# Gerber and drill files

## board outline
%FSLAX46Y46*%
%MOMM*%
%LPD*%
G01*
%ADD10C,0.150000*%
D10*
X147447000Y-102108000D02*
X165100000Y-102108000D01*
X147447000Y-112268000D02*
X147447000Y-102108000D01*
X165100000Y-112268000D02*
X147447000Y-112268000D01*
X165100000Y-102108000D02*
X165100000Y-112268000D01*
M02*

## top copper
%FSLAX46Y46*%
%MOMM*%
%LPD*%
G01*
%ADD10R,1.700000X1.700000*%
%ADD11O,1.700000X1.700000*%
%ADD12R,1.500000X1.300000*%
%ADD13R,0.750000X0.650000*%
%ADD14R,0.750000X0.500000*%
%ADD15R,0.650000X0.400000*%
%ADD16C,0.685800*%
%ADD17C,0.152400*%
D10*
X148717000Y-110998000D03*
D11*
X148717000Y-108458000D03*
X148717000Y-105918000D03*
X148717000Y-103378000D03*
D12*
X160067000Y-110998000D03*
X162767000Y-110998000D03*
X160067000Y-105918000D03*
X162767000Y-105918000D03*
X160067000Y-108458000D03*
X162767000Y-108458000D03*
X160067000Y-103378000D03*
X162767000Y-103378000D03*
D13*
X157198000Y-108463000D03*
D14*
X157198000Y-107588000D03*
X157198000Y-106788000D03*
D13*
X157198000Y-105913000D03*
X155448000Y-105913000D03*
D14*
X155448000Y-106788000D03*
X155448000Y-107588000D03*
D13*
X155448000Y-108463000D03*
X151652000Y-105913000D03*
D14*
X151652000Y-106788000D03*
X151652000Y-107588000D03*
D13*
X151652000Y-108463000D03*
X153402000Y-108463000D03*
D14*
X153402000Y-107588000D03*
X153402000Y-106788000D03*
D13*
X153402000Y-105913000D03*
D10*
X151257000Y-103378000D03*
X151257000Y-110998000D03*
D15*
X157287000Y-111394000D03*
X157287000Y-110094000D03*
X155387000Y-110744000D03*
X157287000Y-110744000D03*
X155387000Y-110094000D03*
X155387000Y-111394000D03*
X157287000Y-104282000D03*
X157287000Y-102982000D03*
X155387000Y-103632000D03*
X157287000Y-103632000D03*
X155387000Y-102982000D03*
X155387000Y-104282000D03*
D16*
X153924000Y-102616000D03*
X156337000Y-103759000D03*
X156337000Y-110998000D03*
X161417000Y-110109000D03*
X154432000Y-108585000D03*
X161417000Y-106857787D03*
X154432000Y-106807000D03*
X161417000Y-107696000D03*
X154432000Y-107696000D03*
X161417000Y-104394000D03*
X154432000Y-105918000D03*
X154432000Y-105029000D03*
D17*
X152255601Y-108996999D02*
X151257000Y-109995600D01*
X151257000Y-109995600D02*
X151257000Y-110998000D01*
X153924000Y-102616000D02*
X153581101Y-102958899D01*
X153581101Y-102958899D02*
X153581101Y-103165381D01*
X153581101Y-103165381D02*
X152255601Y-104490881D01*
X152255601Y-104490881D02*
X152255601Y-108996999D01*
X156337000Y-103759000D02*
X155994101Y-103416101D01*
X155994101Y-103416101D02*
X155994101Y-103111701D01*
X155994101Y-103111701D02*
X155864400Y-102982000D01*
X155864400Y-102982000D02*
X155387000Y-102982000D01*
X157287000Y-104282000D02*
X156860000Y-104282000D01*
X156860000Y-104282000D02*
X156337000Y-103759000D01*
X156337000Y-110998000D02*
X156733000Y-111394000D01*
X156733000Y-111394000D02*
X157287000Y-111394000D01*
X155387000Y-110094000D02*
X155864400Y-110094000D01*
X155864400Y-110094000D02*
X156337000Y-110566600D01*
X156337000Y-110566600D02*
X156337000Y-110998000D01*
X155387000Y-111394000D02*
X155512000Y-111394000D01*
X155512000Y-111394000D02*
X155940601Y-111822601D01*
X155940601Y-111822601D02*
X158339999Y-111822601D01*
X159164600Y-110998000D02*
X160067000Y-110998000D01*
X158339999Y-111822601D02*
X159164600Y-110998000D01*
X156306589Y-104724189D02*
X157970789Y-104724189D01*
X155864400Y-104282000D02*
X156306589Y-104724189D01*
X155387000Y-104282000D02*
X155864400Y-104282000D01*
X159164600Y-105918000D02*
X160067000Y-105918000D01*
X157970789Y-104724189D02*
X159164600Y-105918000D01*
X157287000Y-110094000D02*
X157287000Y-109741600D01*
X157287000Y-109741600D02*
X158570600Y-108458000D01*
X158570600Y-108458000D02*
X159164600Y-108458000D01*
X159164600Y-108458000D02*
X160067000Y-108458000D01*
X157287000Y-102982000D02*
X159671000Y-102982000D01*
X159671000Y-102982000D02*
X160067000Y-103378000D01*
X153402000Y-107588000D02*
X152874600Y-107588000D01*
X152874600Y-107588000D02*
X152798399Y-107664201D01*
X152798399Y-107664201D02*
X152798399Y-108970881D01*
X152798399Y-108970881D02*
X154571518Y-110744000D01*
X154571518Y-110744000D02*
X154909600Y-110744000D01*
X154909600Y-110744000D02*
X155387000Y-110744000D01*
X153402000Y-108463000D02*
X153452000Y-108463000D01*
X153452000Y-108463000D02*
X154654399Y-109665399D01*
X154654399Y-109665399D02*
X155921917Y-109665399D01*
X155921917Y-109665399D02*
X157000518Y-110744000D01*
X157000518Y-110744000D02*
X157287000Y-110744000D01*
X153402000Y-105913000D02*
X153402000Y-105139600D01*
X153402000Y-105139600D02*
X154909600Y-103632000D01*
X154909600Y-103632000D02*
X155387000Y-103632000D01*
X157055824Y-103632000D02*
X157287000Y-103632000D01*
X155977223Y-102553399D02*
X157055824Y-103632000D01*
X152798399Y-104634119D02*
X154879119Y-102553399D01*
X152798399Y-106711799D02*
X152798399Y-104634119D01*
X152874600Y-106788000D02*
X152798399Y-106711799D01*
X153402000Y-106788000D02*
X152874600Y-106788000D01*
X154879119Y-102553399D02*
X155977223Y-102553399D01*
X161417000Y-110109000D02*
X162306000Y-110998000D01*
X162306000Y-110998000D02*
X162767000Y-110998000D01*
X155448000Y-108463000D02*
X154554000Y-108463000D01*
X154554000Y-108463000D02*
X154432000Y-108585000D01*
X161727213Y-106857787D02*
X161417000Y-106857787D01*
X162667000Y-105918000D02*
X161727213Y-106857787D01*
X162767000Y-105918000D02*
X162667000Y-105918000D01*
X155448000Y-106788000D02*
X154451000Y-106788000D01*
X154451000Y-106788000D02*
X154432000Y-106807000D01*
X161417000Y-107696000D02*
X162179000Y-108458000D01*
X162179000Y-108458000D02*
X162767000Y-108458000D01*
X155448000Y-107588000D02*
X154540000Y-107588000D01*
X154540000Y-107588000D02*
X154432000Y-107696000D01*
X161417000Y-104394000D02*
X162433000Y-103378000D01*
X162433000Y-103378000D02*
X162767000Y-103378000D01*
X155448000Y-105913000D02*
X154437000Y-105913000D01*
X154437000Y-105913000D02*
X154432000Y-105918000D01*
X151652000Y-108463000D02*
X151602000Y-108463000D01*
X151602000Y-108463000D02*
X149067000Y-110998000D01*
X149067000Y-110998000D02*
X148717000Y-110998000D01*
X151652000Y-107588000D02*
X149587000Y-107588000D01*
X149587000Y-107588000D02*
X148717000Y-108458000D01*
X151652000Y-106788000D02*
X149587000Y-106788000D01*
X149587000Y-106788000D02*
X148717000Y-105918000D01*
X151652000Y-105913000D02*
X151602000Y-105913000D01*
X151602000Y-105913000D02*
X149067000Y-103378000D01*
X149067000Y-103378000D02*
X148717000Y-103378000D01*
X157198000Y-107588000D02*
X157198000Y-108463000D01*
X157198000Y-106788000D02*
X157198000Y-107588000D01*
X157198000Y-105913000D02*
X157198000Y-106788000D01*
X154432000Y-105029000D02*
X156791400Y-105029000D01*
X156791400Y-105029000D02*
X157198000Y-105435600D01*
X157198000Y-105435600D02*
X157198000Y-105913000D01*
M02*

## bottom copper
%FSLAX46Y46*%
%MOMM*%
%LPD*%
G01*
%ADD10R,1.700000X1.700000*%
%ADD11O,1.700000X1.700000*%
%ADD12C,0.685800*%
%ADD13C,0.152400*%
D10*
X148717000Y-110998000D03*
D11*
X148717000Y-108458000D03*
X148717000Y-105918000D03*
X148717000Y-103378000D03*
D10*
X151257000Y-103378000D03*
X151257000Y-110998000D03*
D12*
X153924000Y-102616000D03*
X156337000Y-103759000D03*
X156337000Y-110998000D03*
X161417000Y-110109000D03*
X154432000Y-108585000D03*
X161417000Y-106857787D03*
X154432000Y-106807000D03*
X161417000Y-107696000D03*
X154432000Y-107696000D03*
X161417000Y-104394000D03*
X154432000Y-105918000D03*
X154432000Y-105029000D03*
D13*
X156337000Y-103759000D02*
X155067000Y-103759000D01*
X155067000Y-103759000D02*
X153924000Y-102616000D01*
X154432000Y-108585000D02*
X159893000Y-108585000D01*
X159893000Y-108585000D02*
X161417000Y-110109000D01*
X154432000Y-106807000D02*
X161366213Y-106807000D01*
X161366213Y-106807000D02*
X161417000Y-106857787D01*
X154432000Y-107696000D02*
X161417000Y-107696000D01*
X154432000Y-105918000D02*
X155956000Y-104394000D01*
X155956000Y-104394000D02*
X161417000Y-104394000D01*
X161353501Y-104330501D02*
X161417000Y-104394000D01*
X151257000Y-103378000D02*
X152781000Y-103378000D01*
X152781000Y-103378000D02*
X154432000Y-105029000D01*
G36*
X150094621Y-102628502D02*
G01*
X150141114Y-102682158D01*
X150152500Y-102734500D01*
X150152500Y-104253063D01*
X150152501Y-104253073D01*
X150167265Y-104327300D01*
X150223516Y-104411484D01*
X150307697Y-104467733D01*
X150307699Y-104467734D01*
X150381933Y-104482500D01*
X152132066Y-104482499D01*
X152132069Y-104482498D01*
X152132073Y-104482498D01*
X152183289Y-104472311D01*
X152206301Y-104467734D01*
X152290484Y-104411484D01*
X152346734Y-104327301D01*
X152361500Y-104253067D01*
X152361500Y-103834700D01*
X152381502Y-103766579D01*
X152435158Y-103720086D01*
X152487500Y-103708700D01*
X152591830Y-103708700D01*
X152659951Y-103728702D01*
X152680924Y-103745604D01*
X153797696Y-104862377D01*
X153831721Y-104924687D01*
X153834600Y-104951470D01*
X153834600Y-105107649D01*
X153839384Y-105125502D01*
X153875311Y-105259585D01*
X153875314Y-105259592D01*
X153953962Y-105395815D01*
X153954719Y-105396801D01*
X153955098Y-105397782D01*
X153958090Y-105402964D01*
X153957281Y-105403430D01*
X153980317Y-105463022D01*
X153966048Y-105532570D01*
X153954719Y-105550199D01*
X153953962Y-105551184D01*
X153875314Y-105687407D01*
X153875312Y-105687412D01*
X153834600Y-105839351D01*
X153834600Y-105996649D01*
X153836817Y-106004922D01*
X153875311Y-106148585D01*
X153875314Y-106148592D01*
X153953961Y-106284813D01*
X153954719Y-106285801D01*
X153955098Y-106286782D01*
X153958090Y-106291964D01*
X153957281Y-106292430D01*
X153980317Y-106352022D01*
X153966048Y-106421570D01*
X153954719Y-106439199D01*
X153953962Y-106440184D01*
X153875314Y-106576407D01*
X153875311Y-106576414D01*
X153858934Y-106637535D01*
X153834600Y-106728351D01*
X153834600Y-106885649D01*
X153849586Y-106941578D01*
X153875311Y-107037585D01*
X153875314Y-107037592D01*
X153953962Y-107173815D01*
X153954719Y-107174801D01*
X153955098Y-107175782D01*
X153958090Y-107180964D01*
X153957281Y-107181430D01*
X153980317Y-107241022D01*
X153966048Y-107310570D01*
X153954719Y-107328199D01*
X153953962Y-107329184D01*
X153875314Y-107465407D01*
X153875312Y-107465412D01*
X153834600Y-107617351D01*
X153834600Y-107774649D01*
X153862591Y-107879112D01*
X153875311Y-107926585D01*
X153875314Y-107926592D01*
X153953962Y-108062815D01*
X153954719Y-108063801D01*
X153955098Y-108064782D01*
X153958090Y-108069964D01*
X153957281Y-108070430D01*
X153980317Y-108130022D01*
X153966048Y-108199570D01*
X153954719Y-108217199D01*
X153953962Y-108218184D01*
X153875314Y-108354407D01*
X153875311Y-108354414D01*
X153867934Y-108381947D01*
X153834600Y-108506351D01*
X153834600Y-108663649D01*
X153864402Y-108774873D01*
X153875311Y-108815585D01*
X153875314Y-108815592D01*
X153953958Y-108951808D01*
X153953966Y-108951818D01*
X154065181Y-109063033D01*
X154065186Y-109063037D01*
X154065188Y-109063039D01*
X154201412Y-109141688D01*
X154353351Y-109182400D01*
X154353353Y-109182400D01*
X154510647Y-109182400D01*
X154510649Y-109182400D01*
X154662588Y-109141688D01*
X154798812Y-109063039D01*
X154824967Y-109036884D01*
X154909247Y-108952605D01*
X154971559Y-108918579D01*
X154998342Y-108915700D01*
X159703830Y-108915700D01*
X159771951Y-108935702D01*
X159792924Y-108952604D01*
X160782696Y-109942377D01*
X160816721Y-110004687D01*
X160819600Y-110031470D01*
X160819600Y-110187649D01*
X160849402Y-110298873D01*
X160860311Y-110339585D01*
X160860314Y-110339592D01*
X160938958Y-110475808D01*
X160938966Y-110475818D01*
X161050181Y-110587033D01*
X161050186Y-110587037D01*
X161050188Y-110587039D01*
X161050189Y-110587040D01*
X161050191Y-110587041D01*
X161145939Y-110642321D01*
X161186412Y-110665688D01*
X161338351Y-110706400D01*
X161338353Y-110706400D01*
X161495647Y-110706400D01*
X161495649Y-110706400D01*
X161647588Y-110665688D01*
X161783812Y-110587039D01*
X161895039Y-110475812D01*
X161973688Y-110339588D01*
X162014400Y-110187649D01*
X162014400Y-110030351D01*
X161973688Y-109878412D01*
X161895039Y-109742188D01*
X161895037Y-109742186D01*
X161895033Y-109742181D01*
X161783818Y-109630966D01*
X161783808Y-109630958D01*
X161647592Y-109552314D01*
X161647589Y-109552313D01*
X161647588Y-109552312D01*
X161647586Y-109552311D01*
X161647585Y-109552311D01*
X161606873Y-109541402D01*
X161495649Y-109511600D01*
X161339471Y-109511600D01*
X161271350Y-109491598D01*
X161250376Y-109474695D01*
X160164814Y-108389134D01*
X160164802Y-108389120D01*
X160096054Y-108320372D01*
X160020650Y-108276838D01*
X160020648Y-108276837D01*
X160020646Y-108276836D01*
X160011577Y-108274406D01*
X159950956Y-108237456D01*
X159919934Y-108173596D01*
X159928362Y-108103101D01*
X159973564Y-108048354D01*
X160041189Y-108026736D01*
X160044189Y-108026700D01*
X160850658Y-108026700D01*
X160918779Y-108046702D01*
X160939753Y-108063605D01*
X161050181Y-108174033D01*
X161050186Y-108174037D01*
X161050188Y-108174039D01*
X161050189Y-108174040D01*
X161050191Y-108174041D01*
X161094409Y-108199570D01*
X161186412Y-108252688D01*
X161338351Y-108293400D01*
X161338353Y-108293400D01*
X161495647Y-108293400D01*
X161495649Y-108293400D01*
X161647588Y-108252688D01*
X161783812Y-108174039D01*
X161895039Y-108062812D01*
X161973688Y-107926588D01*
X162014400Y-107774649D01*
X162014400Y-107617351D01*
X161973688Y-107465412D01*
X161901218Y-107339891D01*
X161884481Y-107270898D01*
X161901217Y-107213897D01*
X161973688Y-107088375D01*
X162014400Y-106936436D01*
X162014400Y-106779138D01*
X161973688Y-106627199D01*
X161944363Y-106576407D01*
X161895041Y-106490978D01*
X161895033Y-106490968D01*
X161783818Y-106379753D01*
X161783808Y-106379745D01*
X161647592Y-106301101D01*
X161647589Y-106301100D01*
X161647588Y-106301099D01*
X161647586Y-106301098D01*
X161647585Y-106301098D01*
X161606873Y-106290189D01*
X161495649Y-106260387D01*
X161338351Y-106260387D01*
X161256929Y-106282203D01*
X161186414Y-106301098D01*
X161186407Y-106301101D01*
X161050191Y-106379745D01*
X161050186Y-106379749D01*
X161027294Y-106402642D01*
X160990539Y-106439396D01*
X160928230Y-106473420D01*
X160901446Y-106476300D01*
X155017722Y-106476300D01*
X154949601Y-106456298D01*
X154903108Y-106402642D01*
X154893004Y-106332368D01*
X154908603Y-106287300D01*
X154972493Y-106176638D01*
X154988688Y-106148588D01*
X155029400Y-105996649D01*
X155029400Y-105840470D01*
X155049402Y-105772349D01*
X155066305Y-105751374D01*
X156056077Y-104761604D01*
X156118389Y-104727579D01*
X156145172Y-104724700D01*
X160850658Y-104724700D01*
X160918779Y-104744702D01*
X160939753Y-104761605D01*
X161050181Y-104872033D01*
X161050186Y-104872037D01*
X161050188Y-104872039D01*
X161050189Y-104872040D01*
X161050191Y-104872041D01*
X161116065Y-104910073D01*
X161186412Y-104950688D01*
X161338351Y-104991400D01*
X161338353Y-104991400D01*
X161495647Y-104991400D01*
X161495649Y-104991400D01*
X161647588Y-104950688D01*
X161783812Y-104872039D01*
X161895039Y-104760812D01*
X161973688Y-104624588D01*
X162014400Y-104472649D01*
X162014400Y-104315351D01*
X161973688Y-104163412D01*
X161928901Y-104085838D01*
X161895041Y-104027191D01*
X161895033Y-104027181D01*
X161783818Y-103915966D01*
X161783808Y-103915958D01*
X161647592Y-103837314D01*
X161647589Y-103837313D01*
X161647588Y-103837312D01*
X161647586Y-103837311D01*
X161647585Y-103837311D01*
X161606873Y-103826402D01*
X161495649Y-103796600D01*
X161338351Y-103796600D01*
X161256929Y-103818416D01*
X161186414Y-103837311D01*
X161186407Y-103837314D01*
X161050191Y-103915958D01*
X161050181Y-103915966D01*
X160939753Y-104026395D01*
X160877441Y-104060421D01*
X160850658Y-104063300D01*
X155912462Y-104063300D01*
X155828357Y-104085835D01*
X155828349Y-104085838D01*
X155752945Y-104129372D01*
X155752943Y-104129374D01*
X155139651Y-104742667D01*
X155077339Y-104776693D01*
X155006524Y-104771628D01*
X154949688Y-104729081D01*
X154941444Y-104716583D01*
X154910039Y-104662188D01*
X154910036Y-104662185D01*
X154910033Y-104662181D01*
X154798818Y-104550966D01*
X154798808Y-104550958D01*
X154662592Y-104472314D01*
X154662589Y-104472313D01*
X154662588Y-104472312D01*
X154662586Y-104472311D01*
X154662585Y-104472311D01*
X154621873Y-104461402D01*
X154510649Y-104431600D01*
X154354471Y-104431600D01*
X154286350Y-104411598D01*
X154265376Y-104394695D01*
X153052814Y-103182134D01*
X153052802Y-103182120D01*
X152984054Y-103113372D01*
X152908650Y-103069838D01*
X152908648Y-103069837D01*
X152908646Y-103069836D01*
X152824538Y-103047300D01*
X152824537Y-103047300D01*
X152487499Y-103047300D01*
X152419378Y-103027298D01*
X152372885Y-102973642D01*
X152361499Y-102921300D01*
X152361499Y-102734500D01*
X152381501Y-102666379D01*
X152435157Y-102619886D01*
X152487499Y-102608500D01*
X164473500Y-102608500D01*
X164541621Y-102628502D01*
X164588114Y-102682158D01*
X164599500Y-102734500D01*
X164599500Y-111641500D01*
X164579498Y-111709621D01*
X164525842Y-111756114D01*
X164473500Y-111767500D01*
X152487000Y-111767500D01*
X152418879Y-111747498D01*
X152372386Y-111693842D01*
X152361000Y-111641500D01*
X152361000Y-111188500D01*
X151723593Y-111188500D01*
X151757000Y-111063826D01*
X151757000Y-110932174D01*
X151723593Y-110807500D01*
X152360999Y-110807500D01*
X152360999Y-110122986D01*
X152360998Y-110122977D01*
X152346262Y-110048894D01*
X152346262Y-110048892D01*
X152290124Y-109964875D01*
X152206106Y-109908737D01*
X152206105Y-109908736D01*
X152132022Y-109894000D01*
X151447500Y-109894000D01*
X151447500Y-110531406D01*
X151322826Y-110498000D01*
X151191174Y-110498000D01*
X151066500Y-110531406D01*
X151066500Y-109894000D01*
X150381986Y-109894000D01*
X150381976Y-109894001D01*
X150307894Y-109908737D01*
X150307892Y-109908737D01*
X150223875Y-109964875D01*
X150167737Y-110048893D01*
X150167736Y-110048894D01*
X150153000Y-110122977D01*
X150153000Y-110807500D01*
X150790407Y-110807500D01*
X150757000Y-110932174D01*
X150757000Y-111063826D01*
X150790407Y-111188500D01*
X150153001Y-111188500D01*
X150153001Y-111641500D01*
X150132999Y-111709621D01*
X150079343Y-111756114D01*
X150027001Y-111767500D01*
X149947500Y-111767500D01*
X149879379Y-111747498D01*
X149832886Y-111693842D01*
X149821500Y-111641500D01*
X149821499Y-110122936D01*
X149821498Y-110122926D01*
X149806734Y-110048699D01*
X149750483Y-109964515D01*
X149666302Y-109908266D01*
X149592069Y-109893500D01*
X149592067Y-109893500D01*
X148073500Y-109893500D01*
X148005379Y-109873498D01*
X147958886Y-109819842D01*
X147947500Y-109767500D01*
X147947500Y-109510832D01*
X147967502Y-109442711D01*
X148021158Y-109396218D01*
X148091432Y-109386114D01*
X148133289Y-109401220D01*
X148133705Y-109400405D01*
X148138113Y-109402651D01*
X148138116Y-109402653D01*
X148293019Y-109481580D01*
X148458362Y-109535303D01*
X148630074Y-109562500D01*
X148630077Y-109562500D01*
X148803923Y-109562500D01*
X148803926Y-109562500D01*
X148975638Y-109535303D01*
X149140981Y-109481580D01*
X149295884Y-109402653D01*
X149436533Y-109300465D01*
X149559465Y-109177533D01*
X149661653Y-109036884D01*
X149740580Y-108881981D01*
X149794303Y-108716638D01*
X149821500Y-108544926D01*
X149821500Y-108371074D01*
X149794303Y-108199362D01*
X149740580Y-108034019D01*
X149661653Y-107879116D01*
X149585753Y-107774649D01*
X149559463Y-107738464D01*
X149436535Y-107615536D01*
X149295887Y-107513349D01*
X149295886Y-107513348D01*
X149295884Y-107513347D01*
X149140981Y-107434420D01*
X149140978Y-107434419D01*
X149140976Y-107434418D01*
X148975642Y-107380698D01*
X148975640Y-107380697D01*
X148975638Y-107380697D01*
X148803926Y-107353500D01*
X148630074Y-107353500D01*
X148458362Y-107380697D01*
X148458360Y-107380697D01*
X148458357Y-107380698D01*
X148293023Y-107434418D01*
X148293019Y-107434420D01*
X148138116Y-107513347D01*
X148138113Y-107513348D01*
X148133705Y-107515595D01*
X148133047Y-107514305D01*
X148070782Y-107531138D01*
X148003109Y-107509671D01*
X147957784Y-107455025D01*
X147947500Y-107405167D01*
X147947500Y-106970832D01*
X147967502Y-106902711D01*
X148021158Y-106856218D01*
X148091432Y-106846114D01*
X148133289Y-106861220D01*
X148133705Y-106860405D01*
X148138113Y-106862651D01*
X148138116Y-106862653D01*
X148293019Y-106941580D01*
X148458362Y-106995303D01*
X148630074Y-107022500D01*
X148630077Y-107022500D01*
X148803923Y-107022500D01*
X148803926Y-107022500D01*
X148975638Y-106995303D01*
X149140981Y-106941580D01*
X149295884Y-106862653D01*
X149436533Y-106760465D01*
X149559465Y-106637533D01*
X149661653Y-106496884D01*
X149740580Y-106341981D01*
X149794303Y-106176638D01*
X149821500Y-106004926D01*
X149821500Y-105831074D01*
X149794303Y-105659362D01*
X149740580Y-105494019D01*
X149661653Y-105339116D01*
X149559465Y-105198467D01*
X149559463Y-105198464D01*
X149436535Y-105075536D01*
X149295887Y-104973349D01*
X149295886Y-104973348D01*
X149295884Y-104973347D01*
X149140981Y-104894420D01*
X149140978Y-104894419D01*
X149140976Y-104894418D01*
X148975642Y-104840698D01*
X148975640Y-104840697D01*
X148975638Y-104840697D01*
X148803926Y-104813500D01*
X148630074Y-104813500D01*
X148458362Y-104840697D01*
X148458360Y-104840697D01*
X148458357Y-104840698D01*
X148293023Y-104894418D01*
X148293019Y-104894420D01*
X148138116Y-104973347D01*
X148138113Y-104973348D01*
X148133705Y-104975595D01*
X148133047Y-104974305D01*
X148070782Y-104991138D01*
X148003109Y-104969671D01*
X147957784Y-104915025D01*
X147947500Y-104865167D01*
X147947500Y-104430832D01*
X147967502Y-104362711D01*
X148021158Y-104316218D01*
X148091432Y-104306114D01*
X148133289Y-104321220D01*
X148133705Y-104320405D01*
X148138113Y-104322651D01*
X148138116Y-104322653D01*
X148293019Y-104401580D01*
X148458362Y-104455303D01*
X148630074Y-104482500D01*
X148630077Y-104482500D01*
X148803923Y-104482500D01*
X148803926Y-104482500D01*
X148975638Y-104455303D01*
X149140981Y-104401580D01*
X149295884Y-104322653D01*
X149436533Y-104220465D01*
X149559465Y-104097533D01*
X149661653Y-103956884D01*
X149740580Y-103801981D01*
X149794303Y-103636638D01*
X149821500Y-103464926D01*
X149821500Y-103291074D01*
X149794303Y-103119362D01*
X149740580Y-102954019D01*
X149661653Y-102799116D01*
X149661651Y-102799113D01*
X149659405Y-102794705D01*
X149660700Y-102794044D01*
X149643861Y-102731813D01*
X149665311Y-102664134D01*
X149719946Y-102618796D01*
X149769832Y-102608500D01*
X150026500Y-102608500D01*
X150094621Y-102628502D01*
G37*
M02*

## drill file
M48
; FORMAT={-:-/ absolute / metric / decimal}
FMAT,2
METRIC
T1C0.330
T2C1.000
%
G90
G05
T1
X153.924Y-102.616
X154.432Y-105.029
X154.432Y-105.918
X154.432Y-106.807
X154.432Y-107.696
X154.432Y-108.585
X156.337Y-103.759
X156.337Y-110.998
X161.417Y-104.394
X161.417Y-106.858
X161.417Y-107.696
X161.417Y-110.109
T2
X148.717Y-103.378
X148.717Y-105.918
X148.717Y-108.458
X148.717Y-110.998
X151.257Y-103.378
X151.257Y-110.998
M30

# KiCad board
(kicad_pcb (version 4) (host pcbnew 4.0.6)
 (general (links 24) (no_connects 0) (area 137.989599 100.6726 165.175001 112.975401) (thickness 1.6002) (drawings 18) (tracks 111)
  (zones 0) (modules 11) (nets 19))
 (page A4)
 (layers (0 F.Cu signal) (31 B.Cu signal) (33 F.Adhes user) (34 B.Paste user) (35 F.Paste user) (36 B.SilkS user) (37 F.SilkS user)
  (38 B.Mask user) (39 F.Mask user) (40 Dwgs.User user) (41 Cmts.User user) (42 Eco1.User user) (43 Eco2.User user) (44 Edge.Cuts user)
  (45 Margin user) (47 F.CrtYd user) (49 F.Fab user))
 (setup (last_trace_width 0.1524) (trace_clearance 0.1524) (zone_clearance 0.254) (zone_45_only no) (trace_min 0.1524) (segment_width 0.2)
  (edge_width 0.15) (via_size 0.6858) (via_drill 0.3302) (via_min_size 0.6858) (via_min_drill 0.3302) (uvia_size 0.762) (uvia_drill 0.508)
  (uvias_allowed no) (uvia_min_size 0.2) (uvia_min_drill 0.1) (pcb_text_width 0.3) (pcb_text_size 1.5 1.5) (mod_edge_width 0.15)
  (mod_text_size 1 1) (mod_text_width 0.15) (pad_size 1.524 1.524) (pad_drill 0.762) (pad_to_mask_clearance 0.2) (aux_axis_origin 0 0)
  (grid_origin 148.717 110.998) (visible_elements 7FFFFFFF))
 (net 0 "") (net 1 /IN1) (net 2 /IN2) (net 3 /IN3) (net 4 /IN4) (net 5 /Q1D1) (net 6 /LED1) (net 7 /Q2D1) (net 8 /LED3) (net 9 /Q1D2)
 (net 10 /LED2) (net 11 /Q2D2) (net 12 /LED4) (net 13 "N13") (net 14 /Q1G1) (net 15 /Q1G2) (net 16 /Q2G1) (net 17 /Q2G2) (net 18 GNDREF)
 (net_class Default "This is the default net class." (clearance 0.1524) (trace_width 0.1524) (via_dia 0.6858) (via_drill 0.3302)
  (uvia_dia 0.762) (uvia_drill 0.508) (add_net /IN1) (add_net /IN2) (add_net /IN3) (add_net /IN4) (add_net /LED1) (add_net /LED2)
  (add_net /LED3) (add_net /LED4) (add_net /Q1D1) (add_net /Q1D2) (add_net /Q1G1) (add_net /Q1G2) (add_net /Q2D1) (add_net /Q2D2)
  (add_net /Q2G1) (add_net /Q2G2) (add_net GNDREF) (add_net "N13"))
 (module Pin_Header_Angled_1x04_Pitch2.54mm (layer F.Cu) (at 148.717 110.998 180)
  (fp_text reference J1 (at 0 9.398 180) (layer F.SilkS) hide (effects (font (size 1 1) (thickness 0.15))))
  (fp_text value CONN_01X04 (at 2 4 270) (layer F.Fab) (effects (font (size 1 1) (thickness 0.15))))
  (pad 1 thru_hole rect (at 0 0 180) (size 1.7 1.7) (drill 1) (layers *.Cu *.Mask) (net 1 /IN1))
  (pad 2 thru_hole oval (at 0 2.54 180) (size 1.7 1.7) (drill 1) (layers *.Cu *.Mask) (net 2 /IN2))
  (pad 3 thru_hole oval (at 0 5.08 180) (size 1.7 1.7) (drill 1) (layers *.Cu *.Mask) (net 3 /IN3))
  (pad 4 thru_hole oval (at 0 7.62 180) (size 1.7 1.7) (drill 1) (layers *.Cu *.Mask) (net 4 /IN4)))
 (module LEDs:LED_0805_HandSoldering (layer F.Cu) (at 161.417 110.998)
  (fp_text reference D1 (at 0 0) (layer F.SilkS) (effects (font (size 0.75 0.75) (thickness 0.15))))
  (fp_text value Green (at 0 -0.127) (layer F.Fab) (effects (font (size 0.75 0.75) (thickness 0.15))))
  (pad 1 smd rect (at -1.35 0) (size 1.5 1.3) (layers F.Cu F.Paste F.Mask) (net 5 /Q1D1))
  (pad 2 smd rect (at 1.35 0) (size 1.5 1.3) (layers F.Cu F.Paste F.Mask) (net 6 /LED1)))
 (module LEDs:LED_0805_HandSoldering (layer F.Cu) (at 161.417 105.918)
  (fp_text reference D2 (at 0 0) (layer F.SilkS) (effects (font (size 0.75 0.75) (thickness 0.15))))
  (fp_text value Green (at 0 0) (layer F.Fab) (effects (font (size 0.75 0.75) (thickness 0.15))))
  (pad 1 smd rect (at -1.35 0) (size 1.5 1.3) (layers F.Cu F.Paste F.Mask) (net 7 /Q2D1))
  (pad 2 smd rect (at 1.35 0) (size 1.5 1.3) (layers F.Cu F.Paste F.Mask) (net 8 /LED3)))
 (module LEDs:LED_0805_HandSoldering (layer F.Cu) (at 161.417 108.458)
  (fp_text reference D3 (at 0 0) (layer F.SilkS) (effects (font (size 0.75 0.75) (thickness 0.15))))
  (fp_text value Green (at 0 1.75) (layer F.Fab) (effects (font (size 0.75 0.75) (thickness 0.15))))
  (pad 1 smd rect (at -1.35 0) (size 1.5 1.3) (layers F.Cu F.Paste F.Mask) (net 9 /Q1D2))
  (pad 2 smd rect (at 1.35 0) (size 1.5 1.3) (layers F.Cu F.Paste F.Mask) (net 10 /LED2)))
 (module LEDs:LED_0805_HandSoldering (layer F.Cu) (at 161.417 103.378)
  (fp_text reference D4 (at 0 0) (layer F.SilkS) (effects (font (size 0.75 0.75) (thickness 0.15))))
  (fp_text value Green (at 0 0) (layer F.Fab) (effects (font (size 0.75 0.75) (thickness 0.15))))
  (pad 1 smd rect (at -1.35 0) (size 1.5 1.3) (layers F.Cu F.Paste F.Mask) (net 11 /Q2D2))
  (pad 2 smd rect (at 1.35 0) (size 1.5 1.3) (layers F.Cu F.Paste F.Mask) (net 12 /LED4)))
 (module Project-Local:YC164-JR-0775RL (layer F.Cu) (at 156.323 107.188 180)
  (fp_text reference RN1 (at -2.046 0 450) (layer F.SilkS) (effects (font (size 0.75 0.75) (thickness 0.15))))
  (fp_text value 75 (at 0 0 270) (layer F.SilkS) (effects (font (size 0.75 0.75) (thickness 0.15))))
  (pad 1 smd rect (at -0.875 -1.275 180) (size 0.75 0.65) (layers F.Cu F.Paste F.Mask) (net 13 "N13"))
  (pad 2 smd rect (at -0.875 -0.4 180) (size 0.75 0.5) (layers F.Cu F.Paste F.Mask) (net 13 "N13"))
  (pad 3 smd rect (at -0.875 0.4 180) (size 0.75 0.5) (layers F.Cu F.Paste F.Mask) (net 13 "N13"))
  (pad 4 smd rect (at -0.875 1.275 180) (size 0.75 0.65) (layers F.Cu F.Paste F.Mask) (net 13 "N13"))
  (pad 5 smd rect (at 0.875 1.275 180) (size 0.75 0.65) (layers F.Cu F.Paste F.Mask) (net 12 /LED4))
  (pad 6 smd rect (at 0.875 0.4 180) (size 0.75 0.5) (layers F.Cu F.Paste F.Mask) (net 8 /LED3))
  (pad 7 smd rect (at 0.875 -0.4 180) (size 0.75 0.5) (layers F.Cu F.Paste F.Mask) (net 10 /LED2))
  (pad 8 smd rect (at 0.875 -1.275 180) (size 0.75 0.65) (layers F.Cu F.Paste F.Mask) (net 6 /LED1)))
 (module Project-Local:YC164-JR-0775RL (layer F.Cu) (at 152.527 107.188)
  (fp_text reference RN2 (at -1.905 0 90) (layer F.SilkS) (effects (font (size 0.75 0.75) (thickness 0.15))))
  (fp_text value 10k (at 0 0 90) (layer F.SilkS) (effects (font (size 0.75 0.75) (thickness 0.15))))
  (pad 1 smd rect (at -0.875 -1.275) (size 0.75 0.65) (layers F.Cu F.Paste F.Mask) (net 4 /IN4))
  (pad 2 smd rect (at -0.875 -0.4) (size 0.75 0.5) (layers F.Cu F.Paste F.Mask) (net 3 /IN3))
  (pad 3 smd rect (at -0.875 0.4) (size 0.75 0.5) (layers F.Cu F.Paste F.Mask) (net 2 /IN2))
  (pad 4 smd rect (at -0.875 1.275) (size 0.75 0.65) (layers F.Cu F.Paste F.Mask) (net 1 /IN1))
  (pad 5 smd rect (at 0.875 1.275) (size 0.75 0.65) (layers F.Cu F.Paste F.Mask) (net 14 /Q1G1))
  (pad 6 smd rect (at 0.875 0.4) (size 0.75 0.5) (layers F.Cu F.Paste F.Mask) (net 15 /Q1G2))
  (pad 7 smd rect (at 0.875 -0.4) (size 0.75 0.5) (layers F.Cu F.Paste F.Mask) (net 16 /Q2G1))
  (pad 8 smd rect (at 0.875 -1.275) (size 0.75 0.65) (layers F.Cu F.Paste F.Mask) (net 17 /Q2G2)))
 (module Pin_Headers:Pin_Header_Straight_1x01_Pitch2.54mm (layer F.Cu) (at 151.257 103.378)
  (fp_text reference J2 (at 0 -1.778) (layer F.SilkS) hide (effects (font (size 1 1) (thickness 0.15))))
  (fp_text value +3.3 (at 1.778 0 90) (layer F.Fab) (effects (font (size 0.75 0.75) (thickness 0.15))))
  (pad 1 thru_hole rect (at 0 0) (size 1.7 1.7) (drill 1) (layers *.Cu *.Mask) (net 13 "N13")))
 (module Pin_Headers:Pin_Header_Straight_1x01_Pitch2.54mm (layer F.Cu) (at 151.257 110.998)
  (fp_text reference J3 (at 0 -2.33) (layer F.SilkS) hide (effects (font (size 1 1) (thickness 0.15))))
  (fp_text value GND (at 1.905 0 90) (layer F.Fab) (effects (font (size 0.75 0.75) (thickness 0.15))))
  (pad 1 thru_hole rect (at 0 0) (size 1.7 1.7) (drill 1) (layers *.Cu *.Mask) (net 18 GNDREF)))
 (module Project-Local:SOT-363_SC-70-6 (layer F.Cu) (at 156.337 110.744 180)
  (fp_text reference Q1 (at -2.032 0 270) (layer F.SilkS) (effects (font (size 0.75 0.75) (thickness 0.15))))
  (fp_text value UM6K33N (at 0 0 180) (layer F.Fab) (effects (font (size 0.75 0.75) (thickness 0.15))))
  (pad 1 smd rect (at -0.95 -0.65 180) (size 0.65 0.4) (layers F.Cu F.Paste F.Mask) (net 18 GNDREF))
  (pad 3 smd rect (at -0.95 0.65 180) (size 0.65 0.4) (layers F.Cu F.Paste F.Mask) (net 9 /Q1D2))
  (pad 5 smd rect (at 0.95 0 180) (size 0.65 0.4) (layers F.Cu F.Paste F.Mask) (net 15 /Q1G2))
  (pad 2 smd rect (at -0.95 0 180) (size 0.65 0.4) (layers F.Cu F.Paste F.Mask) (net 14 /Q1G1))
  (pad 4 smd rect (at 0.95 0.65 180) (size 0.65 0.4) (layers F.Cu F.Paste F.Mask) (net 18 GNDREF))
  (pad 6 smd rect (at 0.95 -0.65 180) (size 0.65 0.4) (layers F.Cu F.Paste F.Mask) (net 5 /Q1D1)))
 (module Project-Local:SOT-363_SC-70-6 (layer F.Cu) (at 156.337 103.632 180)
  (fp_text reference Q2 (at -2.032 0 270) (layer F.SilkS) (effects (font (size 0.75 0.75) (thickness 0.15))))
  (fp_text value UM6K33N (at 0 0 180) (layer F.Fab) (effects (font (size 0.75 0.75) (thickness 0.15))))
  (pad 1 smd rect (at -0.95 -0.65 180) (size 0.65 0.4) (layers F.Cu F.Paste F.Mask) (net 18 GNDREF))
  (pad 3 smd rect (at -0.95 0.65 180) (size 0.65 0.4) (layers F.Cu F.Paste F.Mask) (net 11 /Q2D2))
  (pad 5 smd rect (at 0.95 0 180) (size 0.65 0.4) (layers F.Cu F.Paste F.Mask) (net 17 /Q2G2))
  (pad 2 smd rect (at -0.95 0 180) (size 0.65 0.4) (layers F.Cu F.Paste F.Mask) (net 16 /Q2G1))
  (pad 4 smd rect (at 0.95 0.65 180) (size 0.65 0.4) (layers F.Cu F.Paste F.Mask) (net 18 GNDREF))
  (pad 6 smd rect (at 0.95 -0.65 180) (size 0.65 0.4) (layers F.Cu F.Paste F.Mask) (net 7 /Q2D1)))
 (gr_line (start 147.447 102.108) (end 165.1 102.108) (layer Edge.Cuts) (width 0.15))
 (gr_line (start 147.447 112.268) (end 147.447 102.108) (layer Edge.Cuts) (width 0.15))
 (gr_line (start 165.1 112.268) (end 147.447 112.268) (layer Edge.Cuts) (width 0.15))
 (gr_line (start 165.1 102.108) (end 165.1 112.268) (layer Edge.Cuts) (width 0.15))
 (segment (start 152.255601 108.996999) (end 151.257 109.9956) (width 0.1524) (layer F.Cu) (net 18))
 (segment (start 151.257 109.9956) (end 151.257 110.998) (width 0.1524) (layer F.Cu) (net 18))
 (segment (start 153.924 102.616) (end 153.581101 102.958899) (width 0.1524) (layer F.Cu) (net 18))
 (segment (start 153.581101 102.958899) (end 153.581101 103.165381) (width 0.1524) (layer F.Cu) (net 18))
 (segment (start 153.581101 103.165381) (end 152.255601 104.490881) (width 0.1524) (layer F.Cu) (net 18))
 (segment (start 152.255601 104.490881) (end 152.255601 108.996999) (width 0.1524) (layer F.Cu) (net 18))
 (segment (start 156.337 103.759) (end 155.067 103.759) (width 0.1524) (layer B.Cu) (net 18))
 (segment (start 155.067 103.759) (end 153.924 102.616) (width 0.1524) (layer B.Cu) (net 18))
 (via (at 153.924 102.616) (size 0.6858) (drill 0.3302) (layers F.Cu B.Cu) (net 18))
 (segment (start 156.337 103.759) (end 155.994101 103.416101) (width 0.1524) (layer F.Cu) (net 18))
 (segment (start 155.994101 103.416101) (end 155.994101 103.111701) (width 0.1524) (layer F.Cu) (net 18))
 (segment (start 155.994101 103.111701) (end 155.8644 102.982) (width 0.1524) (layer F.Cu) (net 18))
 (segment (start 155.8644 102.982) (end 155.387 102.982) (width 0.1524) (layer F.Cu) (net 18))
 (segment (start 157.287 104.282) (end 156.86 104.282) (width 0.1524) (layer F.Cu) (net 18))
 (segment (start 156.86 104.282) (end 156.337 103.759) (width 0.1524) (layer F.Cu) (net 18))
 (via (at 156.337 103.759) (size 0.6858) (drill 0.3302) (layers F.Cu B.Cu) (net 18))
 (segment (start 156.337 110.998) (end 156.733 111.394) (width 0.1524) (layer F.Cu) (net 18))
 (segment (start 156.733 111.394) (end 157.287 111.394) (width 0.1524) (layer F.Cu) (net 18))
 (via (at 156.337 110.998) (size 0.6858) (drill 0.3302) (layers F.Cu B.Cu) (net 18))
 (segment (start 155.387 110.094) (end 155.8644 110.094) (width 0.1524) (layer F.Cu) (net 18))
 (segment (start 155.8644 110.094) (end 156.337 110.5666) (width 0.1524) (layer F.Cu) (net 18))
 (segment (start 156.337 110.5666) (end 156.337 110.998) (width 0.1524) (layer F.Cu) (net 18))
 (segment (start 155.387 111.394) (end 155.512 111.394) (width 0.1524) (layer F.Cu) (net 5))
 (segment (start 155.512 111.394) (end 155.940601 111.822601) (width 0.1524) (layer F.Cu) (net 5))
 (segment (start 155.940601 111.822601) (end 158.339999 111.822601) (width 0.1524) (layer F.Cu) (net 5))
 (segment (start 159.1646 110.998) (end 160.067 110.998) (width 0.1524) (layer F.Cu) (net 5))
 (segment (start 158.339999 111.822601) (end 159.1646 110.998) (width 0.1524) (layer F.Cu) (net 5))
 (segment (start 156.306589 104.724189) (end 157.970789 104.724189) (width 0.1524) (layer F.Cu) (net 7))
 (segment (start 155.8644 104.282) (end 156.306589 104.724189) (width 0.1524) (layer F.Cu) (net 7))
 (segment (start 155.387 104.282) (end 155.8644 104.282) (width 0.1524) (layer F.Cu) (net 7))
 (segment (start 159.1646 105.918) (end 160.067 105.918) (width 0.1524) (layer F.Cu) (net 7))
 (segment (start 157.970789 104.724189) (end 159.1646 105.918) (width 0.1524) (layer F.Cu) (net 7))
 (segment (start 157.287 110.094) (end 157.287 109.7416) (width 0.1524) (layer F.Cu) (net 9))
 (segment (start 157.287 109.7416) (end 158.5706 108.458) (width 0.1524) (layer F.Cu) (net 9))
 (segment (start 158.5706 108.458) (end 159.1646 108.458) (width 0.1524) (layer F.Cu) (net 9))
 (segment (start 159.1646 108.458) (end 160.067 108.458) (width 0.1524) (layer F.Cu) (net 9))
 (segment (start 157.287 102.982) (end 159.671 102.982) (width 0.1524) (layer F.Cu) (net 11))
 (segment (start 159.671 102.982) (end 160.067 103.378) (width 0.1524) (layer F.Cu) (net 11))
 (segment (start 153.402 107.588) (end 152.8746 107.588) (width 0.1524) (layer F.Cu) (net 15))
 (segment (start 152.8746 107.588) (end 152.798399 107.664201) (width 0.1524) (layer F.Cu) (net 15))
 (segment (start 152.798399 107.664201) (end 152.798399 108.970881) (width 0.1524) (layer F.Cu) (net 15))
 (segment (start 152.798399 108.970881) (end 154.571518 110.744) (width 0.1524) (layer F.Cu) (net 15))
 (segment (start 154.571518 110.744) (end 154.9096 110.744) (width 0.1524) (layer F.Cu) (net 15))
 (segment (start 154.9096 110.744) (end 155.387 110.744) (width 0.1524) (layer F.Cu) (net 15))
 (segment (start 153.402 108.463) (end 153.452 108.463) (width 0.1524) (layer F.Cu) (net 14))
 (segment (start 153.452 108.463) (end 154.654399 109.665399) (width 0.1524) (layer F.Cu) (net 14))
 (segment (start 154.654399 109.665399) (end 155.921917 109.665399) (width 0.1524) (layer F.Cu) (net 14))
 (segment (start 155.921917 109.665399) (end 157.000518 110.744) (width 0.1524) (layer F.Cu) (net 14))
 (segment (start 157.000518 110.744) (end 157.287 110.744) (width 0.1524) (layer F.Cu) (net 14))
 (segment (start 153.402 105.913) (end 153.402 105.1396) (width 0.1524) (layer F.Cu) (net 17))
 (segment (start 153.402 105.1396) (end 154.9096 103.632) (width 0.1524) (layer F.Cu) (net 17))
 (segment (start 154.9096 103.632) (end 155.387 103.632) (width 0.1524) (layer F.Cu) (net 17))
 (segment (start 157.055824 103.632) (end 157.287 103.632) (width 0.1524) (layer F.Cu) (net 16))
 (segment (start 155.977223 102.553399) (end 157.055824 103.632) (width 0.1524) (layer F.Cu) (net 16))
 (segment (start 152.798399 104.634119) (end 154.879119 102.553399) (width 0.1524) (layer F.Cu) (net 16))
 (segment (start 152.798399 106.711799) (end 152.798399 104.634119) (width 0.1524) (layer F.Cu) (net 16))
 (segment (start 152.8746 106.788) (end 152.798399 106.711799) (width 0.1524) (layer F.Cu) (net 16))
 (segment (start 153.402 106.788) (end 152.8746 106.788) (width 0.1524) (layer F.Cu) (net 16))
 (segment (start 154.879119 102.553399) (end 155.977223 102.553399) (width 0.1524) (layer F.Cu) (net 16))
 (segment (start 161.417 110.109) (end 162.306 110.998) (width 0.1524) (layer F.Cu) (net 6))
 (segment (start 162.306 110.998) (end 162.767 110.998) (width 0.1524) (layer F.Cu) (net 6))
 (segment (start 154.432 108.585) (end 159.893 108.585) (width 0.1524) (layer B.Cu) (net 6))
 (segment (start 159.893 108.585) (end 161.417 110.109) (width 0.1524) (layer B.Cu) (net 6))
 (via (at 161.417 110.109) (size 0.6858) (drill 0.3302) (layers F.Cu B.Cu) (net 6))
 (segment (start 155.448 108.463) (end 154.554 108.463) (width 0.1524) (layer F.Cu) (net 6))
 (segment (start 154.554 108.463) (end 154.432 108.585) (width 0.1524) (layer F.Cu) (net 6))
 (via (at 154.432 108.585) (size 0.6858) (drill 0.3302) (layers F.Cu B.Cu) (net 6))
 (segment (start 161.727213 106.857787) (end 161.417 106.857787) (width 0.1524) (layer F.Cu) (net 8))
 (segment (start 162.667 105.918) (end 161.727213 106.857787) (width 0.1524) (layer F.Cu) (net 8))
 (segment (start 162.767 105.918) (end 162.667 105.918) (width 0.1524) (layer F.Cu) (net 8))
 (segment (start 154.432 106.807) (end 161.366213 106.807) (width 0.1524) (layer B.Cu) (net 8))
 (segment (start 161.366213 106.807) (end 161.417 106.857787) (width 0.1524) (layer B.Cu) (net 8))
 (via (at 161.417 106.857787) (size 0.6858) (drill 0.3302) (layers F.Cu B.Cu) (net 8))
 (segment (start 155.448 106.788) (end 154.451 106.788) (width 0.1524) (layer F.Cu) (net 8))
 (via (at 154.432 106.807) (size 0.6858) (drill 0.3302) (layers F.Cu B.Cu) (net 8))
 (segment (start 154.451 106.788) (end 154.432 106.807) (width 0.1524) (layer F.Cu) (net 8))
 (segment (start 161.417 107.696) (end 162.179 108.458) (width 0.1524) (layer F.Cu) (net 10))
 (segment (start 162.179 108.458) (end 162.767 108.458) (width 0.1524) (layer F.Cu) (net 10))
 (segment (start 154.432 107.696) (end 161.417 107.696) (width 0.1524) (layer B.Cu) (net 10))
 (via (at 161.417 107.696) (size 0.6858) (drill 0.3302) (layers F.Cu B.Cu) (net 10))
 (segment (start 155.448 107.588) (end 154.54 107.588) (width 0.1524) (layer F.Cu) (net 10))
 (segment (start 154.54 107.588) (end 154.432 107.696) (width 0.1524) (layer F.Cu) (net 10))
 (via (at 154.432 107.696) (size 0.6858) (drill 0.3302) (layers F.Cu B.Cu) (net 10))
 (segment (start 154.432 105.918) (end 155.956 104.394) (width 0.1524) (layer B.Cu) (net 12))
 (segment (start 155.956 104.394) (end 161.417 104.394) (width 0.1524) (layer B.Cu) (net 12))
 (segment (start 161.417 104.394) (end 162.433 103.378) (width 0.1524) (layer F.Cu) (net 12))
 (segment (start 162.433 103.378) (end 162.767 103.378) (width 0.1524) (layer F.Cu) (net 12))
 (segment (start 161.353501 104.330501) (end 161.417 104.394) (width 0.1524) (layer B.Cu) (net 12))
 (via (at 161.417 104.394) (size 0.6858) (drill 0.3302) (layers F.Cu B.Cu) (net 12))
 (segment (start 155.448 105.913) (end 154.437 105.913) (width 0.1524) (layer F.Cu) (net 12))
 (segment (start 154.437 105.913) (end 154.432 105.918) (width 0.1524) (layer F.Cu) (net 12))
 (via (at 154.432 105.918) (size 0.6858) (drill 0.3302) (layers F.Cu B.Cu) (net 12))
 (segment (start 151.652 108.463) (end 151.602 108.463) (width 0.1524) (layer F.Cu) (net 1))
 (segment (start 151.602 108.463) (end 149.067 110.998) (width 0.1524) (layer F.Cu) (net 1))
 (segment (start 149.067 110.998) (end 148.717 110.998) (width 0.1524) (layer F.Cu) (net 1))
 (segment (start 151.652 107.588) (end 149.587 107.588) (width 0.1524) (layer F.Cu) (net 2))
 (segment (start 149.587 107.588) (end 148.717 108.458) (width 0.1524) (layer F.Cu) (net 2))
 (segment (start 151.652 106.788) (end 149.587 106.788) (width 0.1524) (layer F.Cu) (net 3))
 (segment (start 149.587 106.788) (end 148.717 105.918) (width 0.1524) (layer F.Cu) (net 3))
 (segment (start 151.652 105.913) (end 151.602 105.913) (width 0.1524) (layer F.Cu) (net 4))
 (segment (start 151.602 105.913) (end 149.067 103.378) (width 0.1524) (layer F.Cu) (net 4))
 (segment (start 149.067 103.378) (end 148.717 103.378) (width 0.1524) (layer F.Cu) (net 4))
 (segment (start 151.257 103.378) (end 152.781 103.378) (width 0.1524) (layer B.Cu) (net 13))
 (segment (start 152.781 103.378) (end 154.432 105.029) (width 0.1524) (layer B.Cu) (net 13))
 (segment (start 157.198 107.588) (end 157.198 108.463) (width 0.1524) (layer F.Cu) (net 13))
 (segment (start 157.198 106.788) (end 157.198 107.588) (width 0.1524) (layer F.Cu) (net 13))
 (segment (start 157.198 105.913) (end 157.198 106.788) (width 0.1524) (layer F.Cu) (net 13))
 (segment (start 154.432 105.029) (end 156.7914 105.029) (width 0.1524) (layer F.Cu) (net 13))
 (segment (start 156.7914 105.029) (end 157.198 105.4356) (width 0.1524) (layer F.Cu) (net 13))
 (segment (start 157.198 105.4356) (end 157.198 105.913) (width 0.1524) (layer F.Cu) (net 13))
 (via (at 154.432 105.029) (size 0.6858) (drill 0.3302) (layers F.Cu B.Cu) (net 13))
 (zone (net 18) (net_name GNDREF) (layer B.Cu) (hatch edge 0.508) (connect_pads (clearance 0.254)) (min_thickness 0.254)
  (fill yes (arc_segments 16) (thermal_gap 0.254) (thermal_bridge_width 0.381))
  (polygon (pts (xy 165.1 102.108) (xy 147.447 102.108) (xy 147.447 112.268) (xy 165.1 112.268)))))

